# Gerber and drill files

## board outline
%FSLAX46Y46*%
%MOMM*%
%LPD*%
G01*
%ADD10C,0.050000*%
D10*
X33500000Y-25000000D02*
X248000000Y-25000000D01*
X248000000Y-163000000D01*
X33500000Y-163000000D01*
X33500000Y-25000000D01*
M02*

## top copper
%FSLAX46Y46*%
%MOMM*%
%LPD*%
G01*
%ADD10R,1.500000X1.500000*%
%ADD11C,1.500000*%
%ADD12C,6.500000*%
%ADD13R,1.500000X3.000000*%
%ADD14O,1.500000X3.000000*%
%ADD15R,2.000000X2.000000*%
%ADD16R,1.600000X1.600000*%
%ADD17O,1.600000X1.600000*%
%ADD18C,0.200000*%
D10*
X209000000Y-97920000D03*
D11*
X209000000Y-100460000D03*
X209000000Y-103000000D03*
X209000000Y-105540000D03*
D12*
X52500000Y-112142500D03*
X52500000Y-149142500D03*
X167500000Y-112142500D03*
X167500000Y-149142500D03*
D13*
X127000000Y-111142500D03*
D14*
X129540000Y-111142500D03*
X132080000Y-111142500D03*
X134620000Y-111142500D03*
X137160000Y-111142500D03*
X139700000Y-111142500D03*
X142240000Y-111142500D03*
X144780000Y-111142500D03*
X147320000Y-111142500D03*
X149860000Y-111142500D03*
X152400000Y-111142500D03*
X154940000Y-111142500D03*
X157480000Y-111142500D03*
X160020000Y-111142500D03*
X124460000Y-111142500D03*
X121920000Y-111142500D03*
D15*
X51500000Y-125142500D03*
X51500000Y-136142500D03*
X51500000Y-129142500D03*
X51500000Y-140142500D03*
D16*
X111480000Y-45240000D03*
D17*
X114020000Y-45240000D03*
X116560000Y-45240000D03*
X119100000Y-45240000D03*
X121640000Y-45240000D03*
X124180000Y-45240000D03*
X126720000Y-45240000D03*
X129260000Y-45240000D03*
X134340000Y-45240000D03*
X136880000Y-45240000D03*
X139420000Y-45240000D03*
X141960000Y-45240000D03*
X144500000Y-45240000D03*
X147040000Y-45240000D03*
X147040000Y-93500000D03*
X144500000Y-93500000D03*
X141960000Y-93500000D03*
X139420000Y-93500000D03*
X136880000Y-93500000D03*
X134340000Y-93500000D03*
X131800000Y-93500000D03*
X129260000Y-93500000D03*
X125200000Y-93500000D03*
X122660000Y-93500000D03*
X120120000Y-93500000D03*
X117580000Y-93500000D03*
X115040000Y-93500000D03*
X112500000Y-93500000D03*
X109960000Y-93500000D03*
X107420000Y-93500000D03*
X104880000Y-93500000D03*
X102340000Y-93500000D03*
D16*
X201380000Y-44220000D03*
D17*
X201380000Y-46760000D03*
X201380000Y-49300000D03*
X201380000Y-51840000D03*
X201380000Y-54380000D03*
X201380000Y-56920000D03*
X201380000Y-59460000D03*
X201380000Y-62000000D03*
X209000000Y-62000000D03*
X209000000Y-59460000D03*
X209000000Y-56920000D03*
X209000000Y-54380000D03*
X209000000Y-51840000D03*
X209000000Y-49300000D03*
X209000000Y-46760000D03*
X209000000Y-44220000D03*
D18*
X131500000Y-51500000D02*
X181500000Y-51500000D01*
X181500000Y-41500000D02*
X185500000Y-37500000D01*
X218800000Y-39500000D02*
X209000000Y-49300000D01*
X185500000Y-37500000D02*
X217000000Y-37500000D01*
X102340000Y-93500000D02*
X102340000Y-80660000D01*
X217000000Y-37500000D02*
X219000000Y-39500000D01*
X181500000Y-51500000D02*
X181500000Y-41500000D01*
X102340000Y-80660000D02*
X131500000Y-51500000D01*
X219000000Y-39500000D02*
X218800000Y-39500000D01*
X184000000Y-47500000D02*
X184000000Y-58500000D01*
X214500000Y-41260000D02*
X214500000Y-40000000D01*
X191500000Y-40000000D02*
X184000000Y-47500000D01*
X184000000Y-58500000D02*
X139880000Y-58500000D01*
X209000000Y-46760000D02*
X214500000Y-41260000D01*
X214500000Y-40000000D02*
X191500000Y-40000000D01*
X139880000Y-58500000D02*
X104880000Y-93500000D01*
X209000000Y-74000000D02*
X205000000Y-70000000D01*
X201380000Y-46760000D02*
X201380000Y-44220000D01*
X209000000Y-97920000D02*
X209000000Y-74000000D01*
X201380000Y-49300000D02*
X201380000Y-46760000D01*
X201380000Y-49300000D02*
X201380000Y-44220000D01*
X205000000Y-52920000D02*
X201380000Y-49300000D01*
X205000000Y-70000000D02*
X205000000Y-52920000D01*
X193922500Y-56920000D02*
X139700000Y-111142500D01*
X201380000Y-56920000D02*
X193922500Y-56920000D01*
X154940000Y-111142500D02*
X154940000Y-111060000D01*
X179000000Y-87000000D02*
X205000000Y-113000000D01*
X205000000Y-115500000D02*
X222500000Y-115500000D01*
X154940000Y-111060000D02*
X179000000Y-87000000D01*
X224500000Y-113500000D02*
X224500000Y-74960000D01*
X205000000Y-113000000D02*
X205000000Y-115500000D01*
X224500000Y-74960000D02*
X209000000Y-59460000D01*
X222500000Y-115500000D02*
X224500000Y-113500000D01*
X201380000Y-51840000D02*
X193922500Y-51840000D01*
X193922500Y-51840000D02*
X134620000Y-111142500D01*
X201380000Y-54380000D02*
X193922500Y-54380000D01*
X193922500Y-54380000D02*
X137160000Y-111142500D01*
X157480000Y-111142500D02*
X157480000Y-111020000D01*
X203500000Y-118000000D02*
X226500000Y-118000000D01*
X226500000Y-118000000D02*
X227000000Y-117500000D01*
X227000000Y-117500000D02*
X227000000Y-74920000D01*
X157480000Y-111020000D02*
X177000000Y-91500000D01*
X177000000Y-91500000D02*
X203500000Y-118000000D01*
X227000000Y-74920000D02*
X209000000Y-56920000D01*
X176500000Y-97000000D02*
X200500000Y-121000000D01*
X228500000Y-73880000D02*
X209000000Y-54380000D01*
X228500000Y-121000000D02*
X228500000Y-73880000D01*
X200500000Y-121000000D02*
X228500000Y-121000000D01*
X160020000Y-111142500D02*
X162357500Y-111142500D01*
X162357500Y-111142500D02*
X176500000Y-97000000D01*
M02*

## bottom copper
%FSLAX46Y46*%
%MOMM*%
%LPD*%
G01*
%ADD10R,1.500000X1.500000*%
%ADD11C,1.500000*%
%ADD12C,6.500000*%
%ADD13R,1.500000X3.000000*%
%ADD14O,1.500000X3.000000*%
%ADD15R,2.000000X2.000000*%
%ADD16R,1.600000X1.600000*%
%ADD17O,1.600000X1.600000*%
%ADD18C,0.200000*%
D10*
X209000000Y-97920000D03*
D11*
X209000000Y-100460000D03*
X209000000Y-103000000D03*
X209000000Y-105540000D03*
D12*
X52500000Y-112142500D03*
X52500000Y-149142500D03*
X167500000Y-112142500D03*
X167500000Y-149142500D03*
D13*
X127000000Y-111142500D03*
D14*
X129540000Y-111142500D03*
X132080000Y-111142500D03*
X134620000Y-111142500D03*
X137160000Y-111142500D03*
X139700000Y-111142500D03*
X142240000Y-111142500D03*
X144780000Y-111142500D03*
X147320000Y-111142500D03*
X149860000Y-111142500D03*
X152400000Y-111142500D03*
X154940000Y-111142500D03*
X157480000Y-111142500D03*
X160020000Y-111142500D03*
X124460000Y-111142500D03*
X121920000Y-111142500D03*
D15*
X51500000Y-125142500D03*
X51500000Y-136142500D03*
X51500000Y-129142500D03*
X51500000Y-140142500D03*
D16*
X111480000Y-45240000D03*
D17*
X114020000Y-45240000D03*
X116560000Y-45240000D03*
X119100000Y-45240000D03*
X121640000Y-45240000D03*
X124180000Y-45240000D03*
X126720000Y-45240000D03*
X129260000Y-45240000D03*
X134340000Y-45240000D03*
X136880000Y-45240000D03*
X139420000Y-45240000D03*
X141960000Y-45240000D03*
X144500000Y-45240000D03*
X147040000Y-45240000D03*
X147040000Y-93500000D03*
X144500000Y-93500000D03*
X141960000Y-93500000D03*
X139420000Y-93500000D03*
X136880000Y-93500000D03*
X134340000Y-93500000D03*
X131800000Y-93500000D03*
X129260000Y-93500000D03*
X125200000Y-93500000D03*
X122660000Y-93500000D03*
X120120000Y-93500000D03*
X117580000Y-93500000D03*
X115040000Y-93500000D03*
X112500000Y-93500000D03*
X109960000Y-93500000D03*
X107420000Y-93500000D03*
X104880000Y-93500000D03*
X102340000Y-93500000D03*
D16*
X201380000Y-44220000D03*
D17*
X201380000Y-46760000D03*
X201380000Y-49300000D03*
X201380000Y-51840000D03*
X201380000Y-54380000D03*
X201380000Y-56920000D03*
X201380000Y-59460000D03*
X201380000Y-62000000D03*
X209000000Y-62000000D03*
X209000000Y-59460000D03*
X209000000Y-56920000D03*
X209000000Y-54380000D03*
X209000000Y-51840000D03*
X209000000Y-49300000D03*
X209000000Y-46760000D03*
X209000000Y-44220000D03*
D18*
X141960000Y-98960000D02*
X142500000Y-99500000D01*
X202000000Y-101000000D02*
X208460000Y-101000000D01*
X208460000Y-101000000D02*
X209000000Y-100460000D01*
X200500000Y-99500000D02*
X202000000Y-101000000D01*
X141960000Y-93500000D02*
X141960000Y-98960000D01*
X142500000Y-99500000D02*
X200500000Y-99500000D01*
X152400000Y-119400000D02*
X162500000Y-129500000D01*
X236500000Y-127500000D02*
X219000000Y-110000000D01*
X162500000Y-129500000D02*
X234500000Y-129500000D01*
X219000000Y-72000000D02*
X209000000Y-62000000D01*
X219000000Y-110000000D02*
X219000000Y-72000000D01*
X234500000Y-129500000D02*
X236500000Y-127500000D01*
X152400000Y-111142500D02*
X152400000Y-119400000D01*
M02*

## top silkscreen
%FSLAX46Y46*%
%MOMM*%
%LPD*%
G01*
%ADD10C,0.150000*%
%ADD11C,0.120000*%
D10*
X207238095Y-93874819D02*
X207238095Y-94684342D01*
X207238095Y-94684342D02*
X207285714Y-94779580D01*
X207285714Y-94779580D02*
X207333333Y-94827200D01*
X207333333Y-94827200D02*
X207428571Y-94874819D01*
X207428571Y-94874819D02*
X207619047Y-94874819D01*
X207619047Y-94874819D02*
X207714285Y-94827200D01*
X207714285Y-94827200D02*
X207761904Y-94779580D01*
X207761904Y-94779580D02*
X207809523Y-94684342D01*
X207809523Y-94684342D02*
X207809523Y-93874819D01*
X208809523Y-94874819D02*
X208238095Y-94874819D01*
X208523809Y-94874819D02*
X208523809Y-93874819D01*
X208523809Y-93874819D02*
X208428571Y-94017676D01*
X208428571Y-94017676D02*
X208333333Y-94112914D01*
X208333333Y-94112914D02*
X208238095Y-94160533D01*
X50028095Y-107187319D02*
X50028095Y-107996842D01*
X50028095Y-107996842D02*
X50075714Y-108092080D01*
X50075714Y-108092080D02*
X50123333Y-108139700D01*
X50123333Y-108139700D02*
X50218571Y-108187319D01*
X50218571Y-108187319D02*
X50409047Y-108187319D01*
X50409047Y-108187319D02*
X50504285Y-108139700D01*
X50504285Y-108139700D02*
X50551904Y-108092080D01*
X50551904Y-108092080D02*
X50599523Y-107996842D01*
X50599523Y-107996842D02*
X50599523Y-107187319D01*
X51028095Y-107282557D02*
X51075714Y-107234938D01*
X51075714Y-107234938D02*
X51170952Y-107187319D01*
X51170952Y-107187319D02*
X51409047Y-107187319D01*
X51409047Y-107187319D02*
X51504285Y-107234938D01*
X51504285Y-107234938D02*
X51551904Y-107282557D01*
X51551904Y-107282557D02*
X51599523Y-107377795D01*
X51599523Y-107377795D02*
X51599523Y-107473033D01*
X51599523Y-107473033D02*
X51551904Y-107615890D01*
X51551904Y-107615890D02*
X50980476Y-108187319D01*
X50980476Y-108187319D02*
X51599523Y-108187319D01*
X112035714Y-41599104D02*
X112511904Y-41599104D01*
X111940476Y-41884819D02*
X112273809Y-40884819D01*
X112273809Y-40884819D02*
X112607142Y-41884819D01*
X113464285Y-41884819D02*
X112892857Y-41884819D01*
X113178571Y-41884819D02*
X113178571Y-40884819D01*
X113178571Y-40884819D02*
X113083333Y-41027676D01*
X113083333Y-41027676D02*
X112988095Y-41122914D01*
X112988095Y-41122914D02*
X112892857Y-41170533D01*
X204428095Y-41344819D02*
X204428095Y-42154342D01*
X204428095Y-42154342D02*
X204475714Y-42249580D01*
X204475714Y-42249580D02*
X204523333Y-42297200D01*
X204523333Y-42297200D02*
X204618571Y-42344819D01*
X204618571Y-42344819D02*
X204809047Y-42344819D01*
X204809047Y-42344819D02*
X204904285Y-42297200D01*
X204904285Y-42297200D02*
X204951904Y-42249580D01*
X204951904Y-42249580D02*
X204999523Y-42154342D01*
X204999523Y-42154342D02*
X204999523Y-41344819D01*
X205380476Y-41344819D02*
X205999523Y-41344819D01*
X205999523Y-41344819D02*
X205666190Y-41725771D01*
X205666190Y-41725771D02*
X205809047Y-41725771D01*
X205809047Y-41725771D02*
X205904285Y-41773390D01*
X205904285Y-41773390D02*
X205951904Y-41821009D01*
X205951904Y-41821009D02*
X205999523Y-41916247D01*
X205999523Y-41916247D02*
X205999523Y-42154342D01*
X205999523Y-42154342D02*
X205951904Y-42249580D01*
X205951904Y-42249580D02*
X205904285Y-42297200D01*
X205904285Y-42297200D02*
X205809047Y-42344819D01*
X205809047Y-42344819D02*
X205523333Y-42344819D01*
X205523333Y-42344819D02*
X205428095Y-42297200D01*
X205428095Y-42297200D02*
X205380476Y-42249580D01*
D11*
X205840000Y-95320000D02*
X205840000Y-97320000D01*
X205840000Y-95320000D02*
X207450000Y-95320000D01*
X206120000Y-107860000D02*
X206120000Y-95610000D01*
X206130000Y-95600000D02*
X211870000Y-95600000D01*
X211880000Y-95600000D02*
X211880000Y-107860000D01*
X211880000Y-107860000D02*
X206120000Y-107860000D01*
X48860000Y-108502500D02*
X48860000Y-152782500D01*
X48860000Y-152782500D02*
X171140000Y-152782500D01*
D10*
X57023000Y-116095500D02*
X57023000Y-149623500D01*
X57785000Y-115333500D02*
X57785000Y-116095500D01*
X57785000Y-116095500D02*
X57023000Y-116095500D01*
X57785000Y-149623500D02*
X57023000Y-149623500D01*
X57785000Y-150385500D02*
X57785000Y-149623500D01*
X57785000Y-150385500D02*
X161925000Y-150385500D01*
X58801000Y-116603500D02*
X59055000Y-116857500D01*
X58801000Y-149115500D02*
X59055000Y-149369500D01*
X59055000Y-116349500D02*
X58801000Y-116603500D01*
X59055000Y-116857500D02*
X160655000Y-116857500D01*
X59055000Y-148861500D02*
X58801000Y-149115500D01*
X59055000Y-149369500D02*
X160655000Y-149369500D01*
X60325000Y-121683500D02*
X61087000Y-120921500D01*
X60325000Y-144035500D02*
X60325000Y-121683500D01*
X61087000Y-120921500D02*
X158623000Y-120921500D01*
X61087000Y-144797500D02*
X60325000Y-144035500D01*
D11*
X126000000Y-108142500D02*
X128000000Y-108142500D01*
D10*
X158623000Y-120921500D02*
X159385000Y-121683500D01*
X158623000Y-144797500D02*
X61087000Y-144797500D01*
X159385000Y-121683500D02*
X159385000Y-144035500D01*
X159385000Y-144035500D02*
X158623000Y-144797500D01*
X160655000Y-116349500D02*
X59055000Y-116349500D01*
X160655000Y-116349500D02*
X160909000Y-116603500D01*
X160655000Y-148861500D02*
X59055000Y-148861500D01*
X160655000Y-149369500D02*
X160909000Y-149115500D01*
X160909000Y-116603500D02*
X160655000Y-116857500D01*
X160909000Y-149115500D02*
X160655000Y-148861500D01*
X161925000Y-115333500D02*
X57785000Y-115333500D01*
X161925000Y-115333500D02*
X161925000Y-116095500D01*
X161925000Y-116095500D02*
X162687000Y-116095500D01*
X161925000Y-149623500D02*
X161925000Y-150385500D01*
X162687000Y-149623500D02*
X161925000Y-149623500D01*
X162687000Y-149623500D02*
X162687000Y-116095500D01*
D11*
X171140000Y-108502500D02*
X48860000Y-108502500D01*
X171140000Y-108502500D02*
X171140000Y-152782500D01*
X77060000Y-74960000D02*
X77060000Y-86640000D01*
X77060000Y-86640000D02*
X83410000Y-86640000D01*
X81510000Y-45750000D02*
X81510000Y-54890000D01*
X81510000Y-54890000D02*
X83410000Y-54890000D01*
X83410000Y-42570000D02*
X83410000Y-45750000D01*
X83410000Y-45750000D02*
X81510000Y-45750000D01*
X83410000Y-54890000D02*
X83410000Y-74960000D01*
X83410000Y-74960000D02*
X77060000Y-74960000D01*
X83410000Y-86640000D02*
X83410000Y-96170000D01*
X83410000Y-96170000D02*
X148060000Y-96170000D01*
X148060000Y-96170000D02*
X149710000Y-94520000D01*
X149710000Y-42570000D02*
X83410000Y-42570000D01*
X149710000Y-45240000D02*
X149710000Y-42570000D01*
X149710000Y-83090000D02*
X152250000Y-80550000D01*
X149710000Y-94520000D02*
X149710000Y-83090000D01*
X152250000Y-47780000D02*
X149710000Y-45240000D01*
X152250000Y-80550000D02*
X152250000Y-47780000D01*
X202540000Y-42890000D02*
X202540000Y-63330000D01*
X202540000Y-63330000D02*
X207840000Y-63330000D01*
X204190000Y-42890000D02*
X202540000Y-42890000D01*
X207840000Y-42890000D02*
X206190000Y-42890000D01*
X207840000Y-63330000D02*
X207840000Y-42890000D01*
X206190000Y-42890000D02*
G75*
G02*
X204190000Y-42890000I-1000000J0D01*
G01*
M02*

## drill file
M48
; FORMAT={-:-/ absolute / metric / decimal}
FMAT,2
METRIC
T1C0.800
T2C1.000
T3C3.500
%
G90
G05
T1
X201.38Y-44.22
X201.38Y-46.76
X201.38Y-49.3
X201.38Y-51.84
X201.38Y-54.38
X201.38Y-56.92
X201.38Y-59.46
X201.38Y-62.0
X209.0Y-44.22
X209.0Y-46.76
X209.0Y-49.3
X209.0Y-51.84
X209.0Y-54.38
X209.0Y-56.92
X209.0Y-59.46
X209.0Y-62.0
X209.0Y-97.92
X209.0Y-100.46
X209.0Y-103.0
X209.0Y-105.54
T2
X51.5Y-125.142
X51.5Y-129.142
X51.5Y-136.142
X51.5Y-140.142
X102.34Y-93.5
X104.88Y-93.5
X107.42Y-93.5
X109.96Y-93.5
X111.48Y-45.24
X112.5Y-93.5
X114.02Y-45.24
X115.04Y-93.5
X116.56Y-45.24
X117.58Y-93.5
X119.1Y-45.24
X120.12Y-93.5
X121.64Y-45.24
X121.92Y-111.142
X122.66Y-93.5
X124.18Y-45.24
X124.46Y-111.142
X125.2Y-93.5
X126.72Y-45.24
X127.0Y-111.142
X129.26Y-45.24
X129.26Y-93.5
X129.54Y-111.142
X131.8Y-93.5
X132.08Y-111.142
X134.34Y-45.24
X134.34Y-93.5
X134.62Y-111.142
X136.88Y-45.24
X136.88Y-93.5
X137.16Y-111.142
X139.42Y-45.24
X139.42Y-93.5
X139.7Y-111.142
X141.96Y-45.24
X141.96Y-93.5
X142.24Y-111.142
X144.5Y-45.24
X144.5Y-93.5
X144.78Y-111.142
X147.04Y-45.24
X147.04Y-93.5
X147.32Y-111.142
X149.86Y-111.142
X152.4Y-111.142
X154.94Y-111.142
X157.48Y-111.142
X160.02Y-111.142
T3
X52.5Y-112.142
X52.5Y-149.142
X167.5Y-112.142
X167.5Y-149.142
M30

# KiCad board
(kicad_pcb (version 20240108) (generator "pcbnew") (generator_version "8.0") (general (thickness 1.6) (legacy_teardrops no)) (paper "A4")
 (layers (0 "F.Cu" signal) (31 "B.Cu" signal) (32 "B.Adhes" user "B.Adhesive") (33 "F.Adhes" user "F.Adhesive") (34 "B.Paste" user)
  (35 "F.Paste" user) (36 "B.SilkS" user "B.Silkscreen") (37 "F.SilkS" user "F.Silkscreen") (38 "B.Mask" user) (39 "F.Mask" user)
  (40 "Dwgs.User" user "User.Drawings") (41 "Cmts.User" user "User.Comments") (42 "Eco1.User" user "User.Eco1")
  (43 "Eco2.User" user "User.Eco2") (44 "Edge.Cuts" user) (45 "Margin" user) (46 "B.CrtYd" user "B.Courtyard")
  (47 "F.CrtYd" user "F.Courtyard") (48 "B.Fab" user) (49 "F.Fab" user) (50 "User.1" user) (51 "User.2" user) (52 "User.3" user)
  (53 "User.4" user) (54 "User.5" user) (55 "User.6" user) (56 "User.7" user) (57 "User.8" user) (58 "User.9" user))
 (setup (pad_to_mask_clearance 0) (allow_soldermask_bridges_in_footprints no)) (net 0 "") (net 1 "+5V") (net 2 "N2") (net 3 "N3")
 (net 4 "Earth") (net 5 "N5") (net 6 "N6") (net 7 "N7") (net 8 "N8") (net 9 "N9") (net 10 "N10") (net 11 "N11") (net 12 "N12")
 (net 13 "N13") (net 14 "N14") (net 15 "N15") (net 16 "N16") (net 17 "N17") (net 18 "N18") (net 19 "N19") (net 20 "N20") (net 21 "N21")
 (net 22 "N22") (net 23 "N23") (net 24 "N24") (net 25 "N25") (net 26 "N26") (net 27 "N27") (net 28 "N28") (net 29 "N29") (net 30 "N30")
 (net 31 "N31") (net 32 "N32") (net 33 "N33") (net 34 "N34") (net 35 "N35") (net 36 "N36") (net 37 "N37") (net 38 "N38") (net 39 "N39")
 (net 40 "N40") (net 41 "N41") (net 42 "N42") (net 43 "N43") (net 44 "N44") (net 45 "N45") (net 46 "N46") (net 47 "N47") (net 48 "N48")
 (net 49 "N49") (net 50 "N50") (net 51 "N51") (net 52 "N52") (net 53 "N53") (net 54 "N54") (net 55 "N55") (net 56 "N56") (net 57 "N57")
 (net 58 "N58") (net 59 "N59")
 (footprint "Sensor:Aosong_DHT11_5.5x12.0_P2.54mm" (layer "F.Cu") (at 209 97.92)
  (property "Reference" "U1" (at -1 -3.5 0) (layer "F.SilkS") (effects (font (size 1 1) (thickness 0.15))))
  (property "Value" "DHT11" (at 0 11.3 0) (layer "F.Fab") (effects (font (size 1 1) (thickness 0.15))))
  (fp_line (start -3.16 -2.6) (end -3.16 -0.6) (stroke (width 0.12) (type solid)) (layer "F.SilkS"))
  (fp_line (start -3.16 -2.6) (end -1.55 -2.6) (stroke (width 0.12) (type solid)) (layer "F.SilkS"))
  (fp_line (start -2.88 9.94) (end -2.88 -2.31) (stroke (width 0.12) (type solid)) (layer "F.SilkS"))
  (fp_line (start -2.87 -2.32) (end 2.87 -2.32) (stroke (width 0.12) (type solid)) (layer "F.SilkS"))
  (fp_line (start 2.88 -2.32) (end 2.88 9.94) (stroke (width 0.12) (type solid)) (layer "F.SilkS"))
  (fp_line (start 2.88 9.94) (end -2.88 9.94) (stroke (width 0.12) (type solid)) (layer "F.SilkS"))
  (pad "1" thru_hole rect (at 0 0) (size 1.5 1.5) (drill 0.8) (layers "*.Cu" "*.Mask") (remove_unused_layers no) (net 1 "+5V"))
  (pad "2" thru_hole circle (at 0 2.54) (size 1.5 1.5) (drill 0.8) (layers "*.Cu" "*.Mask") (remove_unused_layers no) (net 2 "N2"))
  (pad "3" thru_hole circle (at 0 5.08) (size 1.5 1.5) (drill 0.8) (layers "*.Cu" "*.Mask") (remove_unused_layers no) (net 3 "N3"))
  (pad "4" thru_hole circle (at 0 7.62) (size 1.5 1.5) (drill 0.8) (layers "*.Cu" "*.Mask") (remove_unused_layers no) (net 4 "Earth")))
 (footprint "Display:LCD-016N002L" (layer "F.Cu") (at 127 111.1425)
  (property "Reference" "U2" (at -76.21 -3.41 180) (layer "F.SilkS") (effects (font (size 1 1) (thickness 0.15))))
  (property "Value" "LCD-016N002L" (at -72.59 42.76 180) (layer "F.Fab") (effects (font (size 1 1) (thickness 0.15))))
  (fp_line (start -78.14 -2.64) (end -78.14 41.64) (stroke (width 0.12) (type solid)) (layer "F.SilkS"))
  (fp_line (start -78.14 41.64) (end 44.14 41.64) (stroke (width 0.12) (type solid)) (layer "F.SilkS"))
  (fp_line (start -69.977 4.953) (end -69.977 38.481) (stroke (width 0.15) (type solid)) (layer "F.SilkS"))
  (fp_line (start -69.215 4.191) (end -69.215 4.953) (stroke (width 0.15) (type solid)) (layer "F.SilkS"))
  (fp_line (start -69.215 4.953) (end -69.977 4.953) (stroke (width 0.15) (type solid)) (layer "F.SilkS"))
  (fp_line (start -69.215 38.481) (end -69.977 38.481) (stroke (width 0.15) (type solid)) (layer "F.SilkS"))
  (fp_line (start -69.215 39.243) (end -69.215 38.481) (stroke (width 0.15) (type solid)) (layer "F.SilkS"))
  (fp_line (start -69.215 39.243) (end 34.925 39.243) (stroke (width 0.15) (type solid)) (layer "F.SilkS"))
  (fp_line (start -68.199 5.461) (end -67.945 5.715) (stroke (width 0.15) (type solid)) (layer "F.SilkS"))
  (fp_line (start -68.199 37.973) (end -67.945 38.227) (stroke (width 0.15) (type solid)) (layer "F.SilkS"))
  (fp_line (start -67.945 5.207) (end -68.199 5.461) (stroke (width 0.15) (type solid)) (layer "F.SilkS"))
  (fp_line (start -67.945 5.715) (end 33.655 5.715) (stroke (width 0.15) (type solid)) (layer "F.SilkS"))
  (fp_line (start -67.945 37.719) (end -68.199 37.973) (stroke (width 0.15) (type solid)) (layer "F.SilkS"))
  (fp_line (start -67.945 38.227) (end 33.655 38.227) (stroke (width 0.15) (type solid)) (layer "F.SilkS"))
  (fp_line (start -66.675 10.541) (end -65.913 9.779) (stroke (width 0.15) (type solid)) (layer "F.SilkS"))
  (fp_line (start -66.675 32.893) (end -66.675 10.541) (stroke (width 0.15) (type solid)) (layer "F.SilkS"))
  (fp_line (start -65.913 9.779) (end 31.623 9.779) (stroke (width 0.15) (type solid)) (layer "F.SilkS"))
  (fp_line (start -65.913 33.655) (end -66.675 32.893) (stroke (width 0.15) (type solid)) (layer "F.SilkS"))
  (fp_line (start -1 -3) (end 1 -3) (stroke (width 0.12) (type solid)) (layer "F.SilkS"))
  (fp_line (start 31.623 9.779) (end 32.385 10.541) (stroke (width 0.15) (type solid)) (layer "F.SilkS"))
  (fp_line (start 31.623 33.655) (end -65.913 33.655) (stroke (width 0.15) (type solid)) (layer "F.SilkS"))
  (fp_line (start 32.385 10.541) (end 32.385 32.893) (stroke (width 0.15) (type solid)) (layer "F.SilkS"))
  (fp_line (start 32.385 32.893) (end 31.623 33.655) (stroke (width 0.15) (type solid)) (layer "F.SilkS"))
  (fp_line (start 33.655 5.207) (end -67.945 5.207) (stroke (width 0.15) (type solid)) (layer "F.SilkS"))
  (fp_line (start 33.655 5.207) (end 33.909 5.461) (stroke (width 0.15) (type solid)) (layer "F.SilkS"))
  (fp_line (start 33.655 37.719) (end -67.945 37.719) (stroke (width 0.15) (type solid)) (layer "F.SilkS"))
  (fp_line (start 33.655 38.227) (end 33.909 37.973) (stroke (width 0.15) (type solid)) (layer "F.SilkS"))
  (fp_line (start 33.909 5.461) (end 33.655 5.715) (stroke (width 0.15) (type solid)) (layer "F.SilkS"))
  (fp_line (start 33.909 37.973) (end 33.655 37.719) (stroke (width 0.15) (type solid)) (layer "F.SilkS"))
  (fp_line (start 34.925 4.191) (end -69.215 4.191) (stroke (width 0.15) (type solid)) (layer "F.SilkS"))
  (fp_line (start 34.925 4.191) (end 34.925 4.953) (stroke (width 0.15) (type solid)) (layer "F.SilkS"))
  (fp_line (start 34.925 4.953) (end 35.687 4.953) (stroke (width 0.15) (type solid)) (layer "F.SilkS"))
  (fp_line (start 34.925 38.481) (end 34.925 39.243) (stroke (width 0.15) (type solid)) (layer "F.SilkS"))
  (fp_line (start 35.687 38.481) (end 34.925 38.481) (stroke (width 0.15) (type solid)) (layer "F.SilkS"))
  (fp_line (start 35.687 38.481) (end 35.687 4.953) (stroke (width 0.15) (type solid)) (layer "F.SilkS"))
  (fp_line (start 44.14 -2.64) (end -78.14 -2.64) (stroke (width 0.12) (type solid)) (layer "F.SilkS"))
  (fp_line (start 44.14 -2.64) (end 44.14 41.64) (stroke (width 0.12) (type solid)) (layer "F.SilkS"))
  (pad "" thru_hole circle (at -74.5 1 180) (size 6.5 6.5) (drill 3.5) (layers "*.Cu" "*.Mask") (remove_unused_layers no))
  (pad "" thru_hole circle (at -74.5 38 180) (size 6.5 6.5) (drill 3.5) (layers "*.Cu" "*.Mask") (remove_unused_layers no))
  (pad "" thru_hole circle (at 40.5 1 180) (size 6.5 6.5) (drill 3.5) (layers "*.Cu" "*.Mask") (remove_unused_layers no))
  (pad "" thru_hole circle (at 40.5 38 180) (size 6.5 6.5) (drill 3.5) (layers "*.Cu" "*.Mask") (remove_unused_layers no))
  (pad "1" thru_hole rect (at 0 0 180) (size 1.5 3) (drill 1) (layers "*.Cu" "*.Mask") (remove_unused_layers no) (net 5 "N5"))
  (pad "2" thru_hole oval (at 2.54 0 180) (size 1.5 3) (drill 1) (layers "*.Cu" "*.Mask") (remove_unused_layers no) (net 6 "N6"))
  (pad "3" thru_hole oval (at 5.08 0 180) (size 1.5 3) (drill 1) (layers "*.Cu" "*.Mask") (remove_unused_layers no) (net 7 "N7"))
  (pad "4" thru_hole oval (at 7.62 0 180) (size 1.5 3) (drill 1) (layers "*.Cu" "*.Mask") (remove_unused_layers no) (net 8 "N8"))
  (pad "5" thru_hole oval (at 10.16 0 180) (size 1.5 3) (drill 1) (layers "*.Cu" "*.Mask") (remove_unused_layers no) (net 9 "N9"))
  (pad "6" thru_hole oval (at 12.7 0 180) (size 1.5 3) (drill 1) (layers "*.Cu" "*.Mask") (remove_unused_layers no) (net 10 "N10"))
  (pad "7" thru_hole oval (at 15.24 0 180) (size 1.5 3) (drill 1) (layers "*.Cu" "*.Mask") (remove_unused_layers no) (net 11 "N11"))
  (pad "8" thru_hole oval (at 17.78 0 180) (size 1.5 3) (drill 1) (layers "*.Cu" "*.Mask") (remove_unused_layers no) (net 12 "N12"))
  (pad "9" thru_hole oval (at 20.32 0 180) (size 1.5 3) (drill 1) (layers "*.Cu" "*.Mask") (remove_unused_layers no) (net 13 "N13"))
  (pad "10" thru_hole oval (at 22.86 0 180) (size 1.5 3) (drill 1) (layers "*.Cu" "*.Mask") (remove_unused_layers no) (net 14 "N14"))
  (pad "11" thru_hole oval (at 25.4 0 180) (size 1.5 3) (drill 1) (layers "*.Cu" "*.Mask") (remove_unused_layers no) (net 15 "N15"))
  (pad "12" thru_hole oval (at 27.94 0 180) (size 1.5 3) (drill 1) (layers "*.Cu" "*.Mask") (remove_unused_layers no) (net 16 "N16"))
  (pad "13" thru_hole oval (at 30.48 0 180) (size 1.5 3) (drill 1) (layers "*.Cu" "*.Mask") (remove_unused_layers no) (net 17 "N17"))
  (pad "14" thru_hole oval (at 33.02 0 180) (size 1.5 3) (drill 1) (layers "*.Cu" "*.Mask") (remove_unused_layers no) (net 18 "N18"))
  (pad "15" thru_hole oval (at -2.54 0 180) (size 1.5 3) (drill 1) (layers "*.Cu" "*.Mask") (remove_unused_layers no) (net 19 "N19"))
  (pad "16" thru_hole oval (at -5.08 0 180) (size 1.5 3) (drill 1) (layers "*.Cu" "*.Mask") (remove_unused_layers no) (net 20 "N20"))
  (pad "A1" thru_hole rect (at -75.5 14 180) (size 2 2) (drill 1) (layers "*.Cu" "*.Mask") (remove_unused_layers no) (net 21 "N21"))
  (pad "A2" thru_hole rect (at -75.5 25 180) (size 2 2) (drill 1) (layers "*.Cu" "*.Mask") (remove_unused_layers no) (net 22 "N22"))
  (pad "K1" thru_hole rect (at -75.5 18 180) (size 2 2) (drill 1) (layers "*.Cu" "*.Mask") (remove_unused_layers no) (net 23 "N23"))
  (pad "K2" thru_hole rect (at -75.5 29 180) (size 2 2) (drill 1) (layers "*.Cu" "*.Mask") (remove_unused_layers no) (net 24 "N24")))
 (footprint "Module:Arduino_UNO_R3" (layer "F.Cu") (at 111.48 45.24)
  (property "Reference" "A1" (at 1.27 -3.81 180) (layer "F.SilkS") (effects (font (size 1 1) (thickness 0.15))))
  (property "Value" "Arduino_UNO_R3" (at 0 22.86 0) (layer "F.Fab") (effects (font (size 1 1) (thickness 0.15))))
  (fp_line (start -34.42 29.72) (end -34.42 41.4) (stroke (width 0.12) (type solid)) (layer "F.SilkS"))
  (fp_line (start -34.42 41.4) (end -28.07 41.4) (stroke (width 0.12) (type solid)) (layer "F.SilkS"))
  (fp_line (start -29.97 0.51) (end -29.97 9.65) (stroke (width 0.12) (type solid)) (layer "F.SilkS"))
  (fp_line (start -29.97 9.65) (end -28.07 9.65) (stroke (width 0.12) (type solid)) (layer "F.SilkS"))
  (fp_line (start -28.07 -2.67) (end -28.07 0.51) (stroke (width 0.12) (type solid)) (layer "F.SilkS"))
  (fp_line (start -28.07 0.51) (end -29.97 0.51) (stroke (width 0.12) (type solid)) (layer "F.SilkS"))
  (fp_line (start -28.07 9.65) (end -28.07 29.72) (stroke (width 0.12) (type solid)) (layer "F.SilkS"))
  (fp_line (start -28.07 29.72) (end -34.42 29.72) (stroke (width 0.12) (type solid)) (layer "F.SilkS"))
  (fp_line (start -28.07 41.4) (end -28.07 50.93) (stroke (width 0.12) (type solid)) (layer "F.SilkS"))
  (fp_line (start -28.07 50.93) (end 36.58 50.93) (stroke (width 0.12) (type solid)) (layer "F.SilkS"))
  (fp_line (start 36.58 50.93) (end 38.23 49.28) (stroke (width 0.12) (type solid)) (layer "F.SilkS"))
  (fp_line (start 38.23 -2.67) (end -28.07 -2.67) (stroke (width 0.12) (type solid)) (layer "F.SilkS"))
  (fp_line (start 38.23 0) (end 38.23 -2.67) (stroke (width 0.12) (type solid)) (layer "F.SilkS"))
  (fp_line (start 38.23 37.85) (end 40.77 35.31) (stroke (width 0.12) (type solid)) (layer "F.SilkS"))
  (fp_line (start 38.23 49.28) (end 38.23 37.85) (stroke (width 0.12) (type solid)) (layer "F.SilkS"))
  (fp_line (start 40.77 2.54) (end 38.23 0) (stroke (width 0.12) (type solid)) (layer "F.SilkS"))
  (fp_line (start 40.77 35.31) (end 40.77 2.54) (stroke (width 0.12) (type solid)) (layer "F.SilkS"))
  (pad "1" thru_hole rect (at 0 0 90) (size 1.6 1.6) (drill 1) (layers "*.Cu" "*.Mask") (remove_unused_layers no) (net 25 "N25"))
  (pad "2" thru_hole oval (at 2.54 0 90) (size 1.6 1.6) (drill 1) (layers "*.Cu" "*.Mask") (remove_unused_layers no) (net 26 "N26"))
  (pad "3" thru_hole oval (at 5.08 0 90) (size 1.6 1.6) (drill 1) (layers "*.Cu" "*.Mask") (remove_unused_layers no) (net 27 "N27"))
  (pad "4" thru_hole oval (at 7.62 0 90) (size 1.6 1.6) (drill 1) (layers "*.Cu" "*.Mask") (remove_unused_layers no) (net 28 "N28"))
  (pad "5" thru_hole oval (at 10.16 0 90) (size 1.6 1.6) (drill 1) (layers "*.Cu" "*.Mask") (remove_unused_layers no) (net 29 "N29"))
  (pad "6" thru_hole oval (at 12.7 0 90) (size 1.6 1.6) (drill 1) (layers "*.Cu" "*.Mask") (remove_unused_layers no) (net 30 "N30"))
  (pad "7" thru_hole oval (at 15.24 0 90) (size 1.6 1.6) (drill 1) (layers "*.Cu" "*.Mask") (remove_unused_layers no) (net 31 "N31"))
  (pad "8" thru_hole oval (at 17.78 0 90) (size 1.6 1.6) (drill 1) (layers "*.Cu" "*.Mask") (remove_unused_layers no) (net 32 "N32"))
  (pad "9" thru_hole oval (at 22.86 0 90) (size 1.6 1.6) (drill 1) (layers "*.Cu" "*.Mask") (remove_unused_layers no) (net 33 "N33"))
  (pad "10" thru_hole oval (at 25.4 0 90) (size 1.6 1.6) (drill 1) (layers "*.Cu" "*.Mask") (remove_unused_layers no) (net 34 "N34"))
  (pad "11" thru_hole oval (at 27.94 0 90) (size 1.6 1.6) (drill 1) (layers "*.Cu" "*.Mask") (remove_unused_layers no) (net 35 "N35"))
  (pad "12" thru_hole oval (at 30.48 0 90) (size 1.6 1.6) (drill 1) (layers "*.Cu" "*.Mask") (remove_unused_layers no) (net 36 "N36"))
  (pad "13" thru_hole oval (at 33.02 0 90) (size 1.6 1.6) (drill 1) (layers "*.Cu" "*.Mask") (remove_unused_layers no) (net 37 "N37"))
  (pad "14" thru_hole oval (at 35.56 0 90) (size 1.6 1.6) (drill 1) (layers "*.Cu" "*.Mask") (remove_unused_layers no) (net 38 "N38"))
  (pad "15" thru_hole oval (at 35.56 48.26 90) (size 1.6 1.6) (drill 1) (layers "*.Cu" "*.Mask") (remove_unused_layers no) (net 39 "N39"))
  (pad "16" thru_hole oval (at 33.02 48.26 90) (size 1.6 1.6) (drill 1) (layers "*.Cu" "*.Mask") (remove_unused_layers no) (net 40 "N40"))
  (pad "17" thru_hole oval (at 30.48 48.26 90) (size 1.6 1.6) (drill 1) (layers "*.Cu" "*.Mask") (remove_unused_layers no) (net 2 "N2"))
  (pad "18" thru_hole oval (at 27.94 48.26 90) (size 1.6 1.6) (drill 1) (layers "*.Cu" "*.Mask") (remove_unused_layers no) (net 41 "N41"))
  (pad "19" thru_hole oval (at 25.4 48.26 90) (size 1.6 1.6) (drill 1) (layers "*.Cu" "*.Mask") (remove_unused_layers no) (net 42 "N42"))
  (pad "20" thru_hole oval (at 22.86 48.26 90) (size 1.6 1.6) (drill 1) (layers "*.Cu" "*.Mask") (remove_unused_layers no) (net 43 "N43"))
  (pad "21" thru_hole oval (at 20.32 48.26 90) (size 1.6 1.6) (drill 1) (layers "*.Cu" "*.Mask") (remove_unused_layers no) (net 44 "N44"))
  (pad "22" thru_hole oval (at 17.78 48.26 90) (size 1.6 1.6) (drill 1) (layers "*.Cu" "*.Mask") (remove_unused_layers no) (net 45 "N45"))
  (pad "23" thru_hole oval (at 13.72 48.26 90) (size 1.6 1.6) (drill 1) (layers "*.Cu" "*.Mask") (remove_unused_layers no) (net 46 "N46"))
  (pad "24" thru_hole oval (at 11.18 48.26 90) (size 1.6 1.6) (drill 1) (layers "*.Cu" "*.Mask") (remove_unused_layers no) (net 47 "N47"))
  (pad "25" thru_hole oval (at 8.64 48.26 90) (size 1.6 1.6) (drill 1) (layers "*.Cu" "*.Mask") (remove_unused_layers no) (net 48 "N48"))
  (pad "26" thru_hole oval (at 6.1 48.26 90) (size 1.6 1.6) (drill 1) (layers "*.Cu" "*.Mask") (remove_unused_layers no) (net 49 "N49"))
  (pad "27" thru_hole oval (at 3.56 48.26 90) (size 1.6 1.6) (drill 1) (layers "*.Cu" "*.Mask") (remove_unused_layers no) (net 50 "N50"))
  (pad "28" thru_hole oval (at 1.02 48.26 90) (size 1.6 1.6) (drill 1) (layers "*.Cu" "*.Mask") (remove_unused_layers no) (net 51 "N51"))
  (pad "29" thru_hole oval (at -1.52 48.26 90) (size 1.6 1.6) (drill 1) (layers "*.Cu" "*.Mask") (remove_unused_layers no) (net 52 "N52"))
  (pad "30" thru_hole oval (at -4.06 48.26 90) (size 1.6 1.6) (drill 1) (layers "*.Cu" "*.Mask") (remove_unused_layers no) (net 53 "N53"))
  (pad "31" thru_hole oval (at -6.6 48.26 90) (size 1.6 1.6) (drill 1) (layers "*.Cu" "*.Mask") (remove_unused_layers no) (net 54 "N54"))
  (pad "32" thru_hole oval (at -9.14 48.26 90) (size 1.6 1.6) (drill 1) (layers "*.Cu" "*.Mask") (remove_unused_layers no) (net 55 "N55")))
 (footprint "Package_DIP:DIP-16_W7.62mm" (layer "F.Cu") (at 201.38 44.22)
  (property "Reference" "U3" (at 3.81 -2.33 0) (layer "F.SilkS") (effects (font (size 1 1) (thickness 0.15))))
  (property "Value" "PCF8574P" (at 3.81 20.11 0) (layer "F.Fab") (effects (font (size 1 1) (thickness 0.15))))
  (fp_line (start 1.16 -1.33) (end 1.16 19.11) (stroke (width 0.12) (type solid)) (layer "F.SilkS"))
  (fp_line (start 1.16 19.11) (end 6.46 19.11) (stroke (width 0.12) (type solid)) (layer "F.SilkS"))
  (fp_line (start 2.81 -1.33) (end 1.16 -1.33) (stroke (width 0.12) (type solid)) (layer "F.SilkS"))
  (fp_line (start 6.46 -1.33) (end 4.81 -1.33) (stroke (width 0.12) (type solid)) (layer "F.SilkS"))
  (fp_line (start 6.46 19.11) (end 6.46 -1.33) (stroke (width 0.12) (type solid)) (layer "F.SilkS"))
  (fp_arc (start 4.81 -1.33) (mid 3.81 -0.33) (end 2.81 -1.33) (stroke (width 0.12) (type solid)) (layer "F.SilkS"))
  (pad "1" thru_hole rect (at 0 0) (size 1.6 1.6) (drill 0.8) (layers "*.Cu" "*.Mask") (remove_unused_layers no) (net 1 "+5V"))
  (pad "2" thru_hole oval (at 0 2.54) (size 1.6 1.6) (drill 0.8) (layers "*.Cu" "*.Mask") (remove_unused_layers no) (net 1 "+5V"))
  (pad "3" thru_hole oval (at 0 5.08) (size 1.6 1.6) (drill 0.8) (layers "*.Cu" "*.Mask") (remove_unused_layers no) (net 1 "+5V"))
  (pad "4" thru_hole oval (at 0 7.62) (size 1.6 1.6) (drill 0.8) (layers "*.Cu" "*.Mask") (remove_unused_layers no) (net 8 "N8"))
  (pad "5" thru_hole oval (at 0 10.16) (size 1.6 1.6) (drill 0.8) (layers "*.Cu" "*.Mask") (remove_unused_layers no) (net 9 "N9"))
  (pad "6" thru_hole oval (at 0 12.7) (size 1.6 1.6) (drill 0.8) (layers "*.Cu" "*.Mask") (remove_unused_layers no) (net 10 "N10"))
  (pad "7" thru_hole oval (at 0 15.24) (size 1.6 1.6) (drill 0.8) (layers "*.Cu" "*.Mask") (remove_unused_layers no) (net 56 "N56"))
  (pad "8" thru_hole oval (at 0 17.78) (size 1.6 1.6) (drill 0.8) (layers "*.Cu" "*.Mask") (remove_unused_layers no) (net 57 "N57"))
  (pad "9" thru_hole oval (at 7.62 17.78) (size 1.6 1.6) (drill 0.8) (layers "*.Cu" "*.Mask") (remove_unused_layers no) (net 15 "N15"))
  (pad "10" thru_hole oval (at 7.62 15.24) (size 1.6 1.6) (drill 0.8) (layers "*.Cu" "*.Mask") (remove_unused_layers no) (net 16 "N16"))
  (pad "11" thru_hole oval (at 7.62 12.7) (size 1.6 1.6) (drill 0.8) (layers "*.Cu" "*.Mask") (remove_unused_layers no) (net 17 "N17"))
  (pad "12" thru_hole oval (at 7.62 10.16) (size 1.6 1.6) (drill 0.8) (layers "*.Cu" "*.Mask") (remove_unused_layers no) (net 18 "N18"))
  (pad "13" thru_hole oval (at 7.62 7.62) (size 1.6 1.6) (drill 0.8) (layers "*.Cu" "*.Mask") (remove_unused_layers no) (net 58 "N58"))
  (pad "14" thru_hole oval (at 7.62 5.08) (size 1.6 1.6) (drill 0.8) (layers "*.Cu" "*.Mask") (remove_unused_layers no) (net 55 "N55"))
  (pad "15" thru_hole oval (at 7.62 2.54) (size 1.6 1.6) (drill 0.8) (layers "*.Cu" "*.Mask") (remove_unused_layers no) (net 54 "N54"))
  (pad "16" thru_hole oval (at 7.62 0) (size 1.6 1.6) (drill 0.8) (layers "*.Cu" "*.Mask") (remove_unused_layers no) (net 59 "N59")))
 (gr_rect (start 33.5 25) (end 248 163) (stroke (width 0.05) (type default)) (fill none) (layer "Edge.Cuts"))
 (segment (start 131.5 51.5) (end 181.5 51.5) (width 0.2) (layer "F.Cu") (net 55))
 (segment (start 181.5 41.5) (end 185.5 37.5) (width 0.2) (layer "F.Cu") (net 55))
 (segment (start 218.8 39.5) (end 209 49.3) (width 0.2) (layer "F.Cu") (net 55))
 (segment (start 185.5 37.5) (end 217 37.5) (width 0.2) (layer "F.Cu") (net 55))
 (segment (start 102.34 93.5) (end 102.34 80.66) (width 0.2) (layer "F.Cu") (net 55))
 (segment (start 217 37.5) (end 219 39.5) (width 0.2) (layer "F.Cu") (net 55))
 (segment (start 181.5 51.5) (end 181.5 41.5) (width 0.2) (layer "F.Cu") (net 55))
 (segment (start 102.34 80.66) (end 131.5 51.5) (width 0.2) (layer "F.Cu") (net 55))
 (segment (start 219 39.5) (end 218.8 39.5) (width 0.2) (layer "F.Cu") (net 55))
 (segment (start 184 47.5) (end 184 58.5) (width 0.2) (layer "F.Cu") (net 54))
 (segment (start 214.5 41.26) (end 214.5 40) (width 0.2) (layer "F.Cu") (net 54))
 (segment (start 191.5 40) (end 184 47.5) (width 0.2) (layer "F.Cu") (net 54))
 (segment (start 184 58.5) (end 139.88 58.5) (width 0.2) (layer "F.Cu") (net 54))
 (segment (start 209 46.76) (end 214.5 41.26) (width 0.2) (layer "F.Cu") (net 54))
 (segment (start 214.5 40) (end 191.5 40) (width 0.2) (layer "F.Cu") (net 54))
 (segment (start 139.88 58.5) (end 104.88 93.5) (width 0.2) (layer "F.Cu") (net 54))
 (segment (start 141.96 98.96) (end 142.5 99.5) (width 0.2) (layer "B.Cu") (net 2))
 (segment (start 202 101) (end 208.46 101) (width 0.2) (layer "B.Cu") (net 2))
 (segment (start 208.46 101) (end 209 100.46) (width 0.2) (layer "B.Cu") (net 2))
 (segment (start 200.5 99.5) (end 202 101) (width 0.2) (layer "B.Cu") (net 2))
 (segment (start 141.96 93.5) (end 141.96 98.96) (width 0.2) (layer "B.Cu") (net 2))
 (segment (start 142.5 99.5) (end 200.5 99.5) (width 0.2) (layer "B.Cu") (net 2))
 (segment (start 209 74) (end 205 70) (width 0.2) (layer "F.Cu") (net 1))
 (segment (start 201.38 46.76) (end 201.38 44.22) (width 0.2) (layer "F.Cu") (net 1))
 (segment (start 209 97.92) (end 209 74) (width 0.2) (layer "F.Cu") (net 1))
 (segment (start 201.38 49.3) (end 201.38 46.76) (width 0.2) (layer "F.Cu") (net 1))
 (segment (start 201.38 49.3) (end 201.38 44.22) (width 0.2) (layer "F.Cu") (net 1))
 (segment (start 205 52.92) (end 201.38 49.3) (width 0.2) (layer "F.Cu") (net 1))
 (segment (start 205 70) (end 205 52.92) (width 0.2) (layer "F.Cu") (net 1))
 (segment (start 193.9225 56.92) (end 139.7 111.1425) (width 0.2) (layer "F.Cu") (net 10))
 (segment (start 201.38 56.92) (end 193.9225 56.92) (width 0.2) (layer "F.Cu") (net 10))
 (segment (start 154.94 111.1425) (end 154.94 111.06) (width 0.2) (layer "F.Cu") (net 16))
 (segment (start 179 87) (end 205 113) (width 0.2) (layer "F.Cu") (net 16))
 (segment (start 205 115.5) (end 222.5 115.5) (width 0.2) (layer "F.Cu") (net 16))
 (segment (start 154.94 111.06) (end 179 87) (width 0.2) (layer "F.Cu") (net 16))
 (segment (start 224.5 113.5) (end 224.5 74.96) (width 0.2) (layer "F.Cu") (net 16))
 (segment (start 205 113) (end 205 115.5) (width 0.2) (layer "F.Cu") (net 16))
 (segment (start 224.5 74.96) (end 209 59.46) (width 0.2) (layer "F.Cu") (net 16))
 (segment (start 222.5 115.5) (end 224.5 113.5) (width 0.2) (layer "F.Cu") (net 16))
 (segment (start 152.4 119.4) (end 162.5 129.5) (width 0.2) (layer "B.Cu") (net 15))
 (segment (start 236.5 127.5) (end 219 110) (width 0.2) (layer "B.Cu") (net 15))
 (segment (start 162.5 129.5) (end 234.5 129.5) (width 0.2) (layer "B.Cu") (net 15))
 (segment (start 219 72) (end 209 62) (width 0.2) (layer "B.Cu") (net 15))
 (segment (start 219 110) (end 219 72) (width 0.2) (layer "B.Cu") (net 15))
 (segment (start 234.5 129.5) (end 236.5 127.5) (width 0.2) (layer "B.Cu") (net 15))
 (segment (start 152.4 111.1425) (end 152.4 119.4) (width 0.2) (layer "B.Cu") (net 15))
 (segment (start 201.38 51.84) (end 193.9225 51.84) (width 0.2) (layer "F.Cu") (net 8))
 (segment (start 193.9225 51.84) (end 134.62 111.1425) (width 0.2) (layer "F.Cu") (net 8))
 (segment (start 201.38 54.38) (end 193.9225 54.38) (width 0.2) (layer "F.Cu") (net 9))
 (segment (start 193.9225 54.38) (end 137.16 111.1425) (width 0.2) (layer "F.Cu") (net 9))
 (segment (start 157.48 111.1425) (end 157.48 111.02) (width 0.2) (layer "F.Cu") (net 17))
 (segment (start 203.5 118) (end 226.5 118) (width 0.2) (layer "F.Cu") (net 17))
 (segment (start 226.5 118) (end 227 117.5) (width 0.2) (layer "F.Cu") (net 17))
 (segment (start 227 117.5) (end 227 74.92) (width 0.2) (layer "F.Cu") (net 17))
 (segment (start 157.48 111.02) (end 177 91.5) (width 0.2) (layer "F.Cu") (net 17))
 (segment (start 177 91.5) (end 203.5 118) (width 0.2) (layer "F.Cu") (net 17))
 (segment (start 227 74.92) (end 209 56.92) (width 0.2) (layer "F.Cu") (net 17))
 (segment (start 176.5 97) (end 200.5 121) (width 0.2) (layer "F.Cu") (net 18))
 (segment (start 228.5 73.88) (end 209 54.38) (width 0.2) (layer "F.Cu") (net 18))
 (segment (start 228.5 121) (end 228.5 73.88) (width 0.2) (layer "F.Cu") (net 18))
 (segment (start 200.5 121) (end 228.5 121) (width 0.2) (layer "F.Cu") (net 18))
 (segment (start 160.02 111.1425) (end 162.3575 111.1425) (width 0.2) (layer "F.Cu") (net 18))
 (segment (start 162.3575 111.1425) (end 176.5 97) (width 0.2) (layer "F.Cu") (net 18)))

